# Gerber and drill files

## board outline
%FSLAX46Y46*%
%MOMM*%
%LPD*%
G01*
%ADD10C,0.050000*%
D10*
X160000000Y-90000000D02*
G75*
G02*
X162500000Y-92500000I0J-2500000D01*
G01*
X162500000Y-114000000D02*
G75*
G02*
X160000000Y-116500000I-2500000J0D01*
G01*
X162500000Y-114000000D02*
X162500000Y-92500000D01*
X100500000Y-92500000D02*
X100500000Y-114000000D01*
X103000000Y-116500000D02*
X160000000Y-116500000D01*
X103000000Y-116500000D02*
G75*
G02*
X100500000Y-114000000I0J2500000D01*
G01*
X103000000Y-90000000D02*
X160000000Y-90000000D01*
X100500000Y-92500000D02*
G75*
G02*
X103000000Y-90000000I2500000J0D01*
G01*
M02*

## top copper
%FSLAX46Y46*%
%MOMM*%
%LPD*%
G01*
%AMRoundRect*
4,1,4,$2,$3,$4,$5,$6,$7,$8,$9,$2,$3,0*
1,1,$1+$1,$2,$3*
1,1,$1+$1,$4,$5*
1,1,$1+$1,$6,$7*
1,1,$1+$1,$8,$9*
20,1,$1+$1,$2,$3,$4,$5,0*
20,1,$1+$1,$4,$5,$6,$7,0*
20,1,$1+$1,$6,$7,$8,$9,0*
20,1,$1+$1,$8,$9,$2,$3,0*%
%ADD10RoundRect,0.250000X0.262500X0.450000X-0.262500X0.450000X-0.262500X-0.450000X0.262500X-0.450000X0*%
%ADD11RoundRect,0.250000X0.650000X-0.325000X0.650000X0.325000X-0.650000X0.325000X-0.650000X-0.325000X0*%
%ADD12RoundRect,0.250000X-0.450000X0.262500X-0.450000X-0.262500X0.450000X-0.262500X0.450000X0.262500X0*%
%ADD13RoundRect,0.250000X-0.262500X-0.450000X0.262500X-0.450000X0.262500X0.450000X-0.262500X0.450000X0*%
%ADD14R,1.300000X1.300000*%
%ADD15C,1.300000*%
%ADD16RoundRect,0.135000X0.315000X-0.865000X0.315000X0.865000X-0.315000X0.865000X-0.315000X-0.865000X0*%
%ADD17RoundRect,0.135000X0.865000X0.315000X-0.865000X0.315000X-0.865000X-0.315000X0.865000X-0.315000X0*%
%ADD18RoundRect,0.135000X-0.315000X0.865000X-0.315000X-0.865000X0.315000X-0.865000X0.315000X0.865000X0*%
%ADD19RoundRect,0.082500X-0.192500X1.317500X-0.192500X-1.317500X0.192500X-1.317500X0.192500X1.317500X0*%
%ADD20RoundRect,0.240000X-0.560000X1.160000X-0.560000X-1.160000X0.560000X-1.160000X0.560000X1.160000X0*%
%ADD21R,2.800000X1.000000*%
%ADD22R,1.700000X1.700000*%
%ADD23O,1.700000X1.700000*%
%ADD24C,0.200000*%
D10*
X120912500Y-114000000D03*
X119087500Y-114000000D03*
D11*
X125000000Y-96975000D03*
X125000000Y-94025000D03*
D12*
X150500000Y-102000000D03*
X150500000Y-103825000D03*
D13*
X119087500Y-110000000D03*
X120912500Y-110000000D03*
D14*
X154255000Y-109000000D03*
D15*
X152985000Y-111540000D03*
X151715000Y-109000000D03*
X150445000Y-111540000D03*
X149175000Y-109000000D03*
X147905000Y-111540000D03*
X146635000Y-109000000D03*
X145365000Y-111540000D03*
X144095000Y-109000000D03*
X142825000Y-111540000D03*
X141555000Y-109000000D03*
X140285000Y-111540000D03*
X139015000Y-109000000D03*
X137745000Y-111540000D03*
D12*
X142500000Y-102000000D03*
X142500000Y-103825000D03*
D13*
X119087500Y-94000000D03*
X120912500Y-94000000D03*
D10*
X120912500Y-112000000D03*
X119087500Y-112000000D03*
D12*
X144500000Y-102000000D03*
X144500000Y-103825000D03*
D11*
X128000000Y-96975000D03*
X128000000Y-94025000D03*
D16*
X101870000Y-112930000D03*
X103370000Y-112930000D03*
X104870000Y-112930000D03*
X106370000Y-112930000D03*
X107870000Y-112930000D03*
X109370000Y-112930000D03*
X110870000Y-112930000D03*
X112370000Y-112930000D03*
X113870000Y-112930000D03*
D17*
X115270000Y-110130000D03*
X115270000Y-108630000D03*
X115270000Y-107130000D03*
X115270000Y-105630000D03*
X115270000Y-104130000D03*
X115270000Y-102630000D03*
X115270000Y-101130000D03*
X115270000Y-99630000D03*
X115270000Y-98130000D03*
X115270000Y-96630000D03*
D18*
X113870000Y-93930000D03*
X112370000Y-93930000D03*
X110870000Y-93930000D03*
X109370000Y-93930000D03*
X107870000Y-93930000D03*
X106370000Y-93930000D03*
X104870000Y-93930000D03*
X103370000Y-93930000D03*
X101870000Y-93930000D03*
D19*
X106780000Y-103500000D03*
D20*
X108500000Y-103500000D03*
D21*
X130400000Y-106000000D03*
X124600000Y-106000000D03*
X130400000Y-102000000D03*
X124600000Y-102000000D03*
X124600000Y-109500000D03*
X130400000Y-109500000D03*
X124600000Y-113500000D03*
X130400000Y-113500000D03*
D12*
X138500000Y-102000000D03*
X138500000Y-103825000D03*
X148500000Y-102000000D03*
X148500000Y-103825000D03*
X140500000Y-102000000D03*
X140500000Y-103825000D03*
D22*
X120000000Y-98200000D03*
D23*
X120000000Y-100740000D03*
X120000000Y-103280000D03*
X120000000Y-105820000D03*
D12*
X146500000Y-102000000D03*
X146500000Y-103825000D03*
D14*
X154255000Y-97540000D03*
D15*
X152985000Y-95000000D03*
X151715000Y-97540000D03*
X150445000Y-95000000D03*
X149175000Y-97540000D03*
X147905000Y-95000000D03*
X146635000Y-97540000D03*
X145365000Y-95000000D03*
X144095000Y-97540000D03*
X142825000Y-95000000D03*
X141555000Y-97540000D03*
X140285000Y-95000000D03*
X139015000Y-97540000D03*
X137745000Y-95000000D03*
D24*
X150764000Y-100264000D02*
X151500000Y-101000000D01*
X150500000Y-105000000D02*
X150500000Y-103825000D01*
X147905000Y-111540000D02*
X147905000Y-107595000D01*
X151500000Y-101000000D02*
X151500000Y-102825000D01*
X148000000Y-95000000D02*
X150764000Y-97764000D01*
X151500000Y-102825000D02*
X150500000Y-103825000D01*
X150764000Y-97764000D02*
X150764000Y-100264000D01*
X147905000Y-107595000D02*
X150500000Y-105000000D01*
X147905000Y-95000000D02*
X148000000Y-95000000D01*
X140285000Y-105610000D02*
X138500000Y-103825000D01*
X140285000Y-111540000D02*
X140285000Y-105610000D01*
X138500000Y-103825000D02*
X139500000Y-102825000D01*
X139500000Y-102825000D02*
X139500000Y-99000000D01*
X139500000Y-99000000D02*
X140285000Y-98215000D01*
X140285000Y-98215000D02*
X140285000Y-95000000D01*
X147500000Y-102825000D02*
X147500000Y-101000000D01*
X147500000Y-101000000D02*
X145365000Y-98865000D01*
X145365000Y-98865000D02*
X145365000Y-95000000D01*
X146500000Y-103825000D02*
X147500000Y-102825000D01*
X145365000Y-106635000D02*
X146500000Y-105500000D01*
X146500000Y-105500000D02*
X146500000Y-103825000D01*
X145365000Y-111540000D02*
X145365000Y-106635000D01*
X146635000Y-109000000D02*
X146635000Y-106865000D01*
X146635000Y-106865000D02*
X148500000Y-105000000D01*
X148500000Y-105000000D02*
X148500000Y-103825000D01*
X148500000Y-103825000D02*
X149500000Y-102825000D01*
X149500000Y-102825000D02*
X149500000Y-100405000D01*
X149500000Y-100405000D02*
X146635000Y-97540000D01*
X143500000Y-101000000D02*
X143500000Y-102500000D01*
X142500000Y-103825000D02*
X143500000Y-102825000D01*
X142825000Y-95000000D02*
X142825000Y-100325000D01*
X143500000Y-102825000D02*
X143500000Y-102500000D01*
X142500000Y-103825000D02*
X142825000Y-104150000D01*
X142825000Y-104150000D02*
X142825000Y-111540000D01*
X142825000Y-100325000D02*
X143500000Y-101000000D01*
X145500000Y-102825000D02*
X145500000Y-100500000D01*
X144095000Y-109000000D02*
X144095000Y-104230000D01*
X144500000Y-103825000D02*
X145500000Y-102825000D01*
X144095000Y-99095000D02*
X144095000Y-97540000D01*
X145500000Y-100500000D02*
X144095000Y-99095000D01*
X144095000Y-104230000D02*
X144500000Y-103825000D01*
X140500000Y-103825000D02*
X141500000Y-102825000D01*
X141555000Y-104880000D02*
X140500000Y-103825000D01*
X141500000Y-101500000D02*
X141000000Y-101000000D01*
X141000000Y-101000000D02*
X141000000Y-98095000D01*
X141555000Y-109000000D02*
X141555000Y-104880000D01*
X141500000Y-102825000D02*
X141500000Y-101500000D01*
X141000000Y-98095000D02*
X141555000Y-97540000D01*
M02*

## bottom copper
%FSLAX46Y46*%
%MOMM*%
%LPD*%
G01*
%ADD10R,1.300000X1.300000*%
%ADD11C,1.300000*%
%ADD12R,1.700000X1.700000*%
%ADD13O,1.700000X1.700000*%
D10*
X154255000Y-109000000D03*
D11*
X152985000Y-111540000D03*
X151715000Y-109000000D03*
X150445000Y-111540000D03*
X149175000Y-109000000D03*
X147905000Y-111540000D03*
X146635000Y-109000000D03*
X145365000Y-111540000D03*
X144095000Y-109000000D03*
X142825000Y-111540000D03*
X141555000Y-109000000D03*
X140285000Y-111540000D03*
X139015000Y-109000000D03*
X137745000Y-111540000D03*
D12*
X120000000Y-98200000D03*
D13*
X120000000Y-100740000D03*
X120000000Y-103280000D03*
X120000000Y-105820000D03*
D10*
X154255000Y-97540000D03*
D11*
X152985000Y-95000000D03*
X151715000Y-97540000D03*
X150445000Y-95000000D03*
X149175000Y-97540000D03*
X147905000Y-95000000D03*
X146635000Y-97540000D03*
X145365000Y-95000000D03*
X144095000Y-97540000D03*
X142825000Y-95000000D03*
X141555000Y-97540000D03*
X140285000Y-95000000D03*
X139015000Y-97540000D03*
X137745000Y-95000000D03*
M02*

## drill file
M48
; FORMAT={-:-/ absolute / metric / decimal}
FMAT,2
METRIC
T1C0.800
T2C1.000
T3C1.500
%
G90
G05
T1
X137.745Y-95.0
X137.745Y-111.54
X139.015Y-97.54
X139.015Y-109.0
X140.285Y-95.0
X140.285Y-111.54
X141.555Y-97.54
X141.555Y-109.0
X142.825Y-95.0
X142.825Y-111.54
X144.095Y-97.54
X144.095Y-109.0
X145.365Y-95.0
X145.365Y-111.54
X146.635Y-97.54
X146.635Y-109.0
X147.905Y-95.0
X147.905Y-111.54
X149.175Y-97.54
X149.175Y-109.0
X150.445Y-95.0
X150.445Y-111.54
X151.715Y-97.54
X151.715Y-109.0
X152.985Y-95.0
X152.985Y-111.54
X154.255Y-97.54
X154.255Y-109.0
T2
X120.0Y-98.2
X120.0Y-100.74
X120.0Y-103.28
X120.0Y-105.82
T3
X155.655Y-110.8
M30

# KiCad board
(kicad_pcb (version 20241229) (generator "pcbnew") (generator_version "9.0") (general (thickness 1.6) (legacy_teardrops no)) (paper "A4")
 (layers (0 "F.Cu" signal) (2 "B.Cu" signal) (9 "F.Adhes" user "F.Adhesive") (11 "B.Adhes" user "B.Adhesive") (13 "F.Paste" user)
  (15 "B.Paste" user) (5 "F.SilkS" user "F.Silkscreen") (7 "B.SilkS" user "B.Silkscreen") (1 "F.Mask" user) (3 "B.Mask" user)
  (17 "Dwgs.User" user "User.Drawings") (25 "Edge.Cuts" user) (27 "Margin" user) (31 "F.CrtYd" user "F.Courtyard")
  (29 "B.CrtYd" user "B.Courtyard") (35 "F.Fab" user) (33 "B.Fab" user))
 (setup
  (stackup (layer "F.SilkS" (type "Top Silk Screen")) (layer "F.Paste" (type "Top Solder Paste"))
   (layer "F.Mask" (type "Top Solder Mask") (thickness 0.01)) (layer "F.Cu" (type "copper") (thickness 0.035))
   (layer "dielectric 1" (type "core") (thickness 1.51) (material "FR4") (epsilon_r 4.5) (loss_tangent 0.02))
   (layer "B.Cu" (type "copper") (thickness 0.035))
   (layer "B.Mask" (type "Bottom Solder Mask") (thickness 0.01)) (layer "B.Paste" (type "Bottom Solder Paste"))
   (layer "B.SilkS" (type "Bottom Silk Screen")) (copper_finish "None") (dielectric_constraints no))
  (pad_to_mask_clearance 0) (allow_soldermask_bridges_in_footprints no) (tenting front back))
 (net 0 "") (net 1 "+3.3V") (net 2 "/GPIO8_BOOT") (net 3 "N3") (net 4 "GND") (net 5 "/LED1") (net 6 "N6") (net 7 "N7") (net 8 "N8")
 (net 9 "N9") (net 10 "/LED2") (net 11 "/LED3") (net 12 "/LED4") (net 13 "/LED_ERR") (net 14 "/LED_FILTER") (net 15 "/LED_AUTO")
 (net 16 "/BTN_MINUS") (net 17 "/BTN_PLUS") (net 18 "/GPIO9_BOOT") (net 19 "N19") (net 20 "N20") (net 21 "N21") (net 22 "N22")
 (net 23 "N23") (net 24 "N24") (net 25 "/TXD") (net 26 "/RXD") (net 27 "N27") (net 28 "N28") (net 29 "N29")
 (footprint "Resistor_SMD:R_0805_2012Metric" (layer "F.Cu") (at 120 114 180)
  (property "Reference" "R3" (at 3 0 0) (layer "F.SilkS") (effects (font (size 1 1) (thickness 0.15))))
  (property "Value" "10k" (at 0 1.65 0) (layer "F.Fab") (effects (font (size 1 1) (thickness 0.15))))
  (pad "1" smd roundrect (at -0.9125 0 180) (size 1.025 1.4) (layers "F.Cu" "F.Mask" "F.Paste") (roundrect_rratio 0.243902) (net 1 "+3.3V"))
  (pad "2" smd roundrect (at 0.9125 0 180) (size 1.025 1.4) (layers "F.Cu" "F.Mask" "F.Paste") (roundrect_rratio 0.243902)
   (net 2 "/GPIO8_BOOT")))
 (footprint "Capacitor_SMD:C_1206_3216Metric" (layer "F.Cu") (at 125 95.5 90)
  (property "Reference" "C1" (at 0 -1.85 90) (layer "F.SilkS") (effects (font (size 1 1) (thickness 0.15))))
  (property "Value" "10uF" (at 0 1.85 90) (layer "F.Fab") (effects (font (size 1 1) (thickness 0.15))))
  (pad "1" smd roundrect (at -1.475 0 90) (size 1.15 1.8) (layers "F.Cu" "F.Mask" "F.Paste") (roundrect_rratio 0.217391) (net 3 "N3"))
  (pad "2" smd roundrect (at 1.475 0 90) (size 1.15 1.8) (layers "F.Cu" "F.Mask" "F.Paste") (roundrect_rratio 0.217391) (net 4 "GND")))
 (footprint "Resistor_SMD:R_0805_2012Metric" (layer "F.Cu") (at 150.5 102.9125 -90)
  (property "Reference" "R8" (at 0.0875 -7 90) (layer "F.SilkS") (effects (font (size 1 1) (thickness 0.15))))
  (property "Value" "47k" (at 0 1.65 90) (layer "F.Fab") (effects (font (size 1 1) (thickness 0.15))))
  (pad "1" smd roundrect (at -0.9125 0 270) (size 1.025 1.4) (layers "F.Cu" "F.Mask" "F.Paste") (roundrect_rratio 0.243902) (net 1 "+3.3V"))
  (pad "2" smd roundrect (at 0.9125 0 270) (size 1.025 1.4) (layers "F.Cu" "F.Mask" "F.Paste") (roundrect_rratio 0.243902) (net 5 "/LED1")))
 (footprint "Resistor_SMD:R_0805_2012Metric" (layer "F.Cu") (at 120 110)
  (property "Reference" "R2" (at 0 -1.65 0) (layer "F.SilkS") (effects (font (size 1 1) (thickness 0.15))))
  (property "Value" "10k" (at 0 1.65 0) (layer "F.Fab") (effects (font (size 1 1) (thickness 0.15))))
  (pad "1" smd roundrect (at -0.9125 0) (size 1.025 1.4) (layers "F.Cu" "F.Mask" "F.Paste") (roundrect_rratio 0.243902) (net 1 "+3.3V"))
  (pad "2" smd roundrect (at 0.9125 0) (size 1.025 1.4) (layers "F.Cu" "F.Mask" "F.Paste") (roundrect_rratio 0.243902) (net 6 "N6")))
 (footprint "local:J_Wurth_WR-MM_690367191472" (layer "F.Cu") (at 154.255 109 -90)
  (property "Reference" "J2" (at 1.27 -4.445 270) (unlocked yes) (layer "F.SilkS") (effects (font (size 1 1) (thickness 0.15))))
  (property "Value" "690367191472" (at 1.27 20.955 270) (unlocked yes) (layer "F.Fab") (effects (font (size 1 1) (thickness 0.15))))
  (pad "" np_thru_hole circle (at 1.8 -1.4) (size 1.5 1.5) (drill 1.5) (layers "*.Cu" "*.Mask"))
  (pad "1" thru_hole rect (at 0 0) (size 1.3 1.3) (drill 0.8) (layers "*.Cu" "*.Mask") (remove_unused_layers no) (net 1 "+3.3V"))
  (pad "2" thru_hole circle (at 2.54 1.27) (size 1.3 1.3) (drill 0.8) (layers "*.Cu" "*.Mask") (remove_unused_layers no) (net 4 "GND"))
  (pad "3" thru_hole circle (at 0 2.54) (size 1.3 1.3) (drill 0.8) (layers "*.Cu" "*.Mask") (remove_unused_layers no) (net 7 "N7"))
  (pad "4" thru_hole circle (at 2.54 3.81) (size 1.3 1.3) (drill 0.8) (layers "*.Cu" "*.Mask") (remove_unused_layers no) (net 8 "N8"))
  (pad "5" thru_hole circle (at 0 5.08) (size 1.3 1.3) (drill 0.8) (layers "*.Cu" "*.Mask") (remove_unused_layers no) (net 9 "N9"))
  (pad "6" thru_hole circle (at 2.54 6.35) (size 1.3 1.3) (drill 0.8) (layers "*.Cu" "*.Mask") (remove_unused_layers no) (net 5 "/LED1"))
  (pad "7" thru_hole circle (at 0 7.62) (size 1.3 1.3) (drill 0.8) (layers "*.Cu" "*.Mask") (remove_unused_layers no) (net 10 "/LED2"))
  (pad "8" thru_hole circle (at 2.54 8.89) (size 1.3 1.3) (drill 0.8) (layers "*.Cu" "*.Mask") (remove_unused_layers no) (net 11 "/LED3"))
  (pad "9" thru_hole circle (at 0 10.16) (size 1.3 1.3) (drill 0.8) (layers "*.Cu" "*.Mask") (remove_unused_layers no) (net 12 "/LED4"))
  (pad "10" thru_hole circle (at 2.54 11.43) (size 1.3 1.3) (drill 0.8) (layers "*.Cu" "*.Mask") (remove_unused_layers no)
   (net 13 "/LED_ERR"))
  (pad "11" thru_hole circle (at 0 12.7) (size 1.3 1.3) (drill 0.8) (layers "*.Cu" "*.Mask") (remove_unused_layers no)
   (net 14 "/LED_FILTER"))
  (pad "12" thru_hole circle (at 2.54 13.97) (size 1.3 1.3) (drill 0.8) (layers "*.Cu" "*.Mask") (remove_unused_layers no)
   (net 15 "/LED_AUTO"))
  (pad "13" thru_hole circle (at 0 15.24) (size 1.3 1.3) (drill 0.8) (layers "*.Cu" "*.Mask") (remove_unused_layers no)
   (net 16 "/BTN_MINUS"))
  (pad "14" thru_hole circle (at 2.54 16.51) (size 1.3 1.3) (drill 0.8) (layers "*.Cu" "*.Mask") (remove_unused_layers no)
   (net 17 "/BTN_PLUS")))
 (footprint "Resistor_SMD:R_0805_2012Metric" (layer "F.Cu") (at 142.5 102.9125 -90)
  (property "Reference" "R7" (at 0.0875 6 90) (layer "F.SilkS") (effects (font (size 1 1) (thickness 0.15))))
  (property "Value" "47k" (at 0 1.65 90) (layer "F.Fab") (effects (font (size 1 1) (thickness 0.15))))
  (pad "1" smd roundrect (at -0.9125 0 270) (size 1.025 1.4) (layers "F.Cu" "F.Mask" "F.Paste") (roundrect_rratio 0.243902) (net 1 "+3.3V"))
  (pad "2" smd roundrect (at 0.9125 0 270) (size 1.025 1.4) (layers "F.Cu" "F.Mask" "F.Paste") (roundrect_rratio 0.243902)
   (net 13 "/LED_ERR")))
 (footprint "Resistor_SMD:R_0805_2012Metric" (layer "F.Cu") (at 120 94)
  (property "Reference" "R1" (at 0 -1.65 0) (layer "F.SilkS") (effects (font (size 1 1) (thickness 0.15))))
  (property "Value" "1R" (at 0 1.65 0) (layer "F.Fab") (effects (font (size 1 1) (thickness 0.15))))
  (pad "1" smd roundrect (at -0.9125 0) (size 1.025 1.4) (layers "F.Cu" "F.Mask" "F.Paste") (roundrect_rratio 0.243902) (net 1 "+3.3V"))
  (pad "2" smd roundrect (at 0.9125 0) (size 1.025 1.4) (layers "F.Cu" "F.Mask" "F.Paste") (roundrect_rratio 0.243902) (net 3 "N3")))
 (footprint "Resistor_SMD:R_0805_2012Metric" (layer "F.Cu") (at 120 112 180)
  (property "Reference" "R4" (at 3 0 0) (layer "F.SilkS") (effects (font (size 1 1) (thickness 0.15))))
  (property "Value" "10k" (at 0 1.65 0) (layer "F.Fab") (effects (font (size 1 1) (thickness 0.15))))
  (pad "1" smd roundrect (at -0.9125 0 180) (size 1.025 1.4) (layers "F.Cu" "F.Mask" "F.Paste") (roundrect_rratio 0.243902) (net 1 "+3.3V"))
  (pad "2" smd roundrect (at 0.9125 0 180) (size 1.025 1.4) (layers "F.Cu" "F.Mask" "F.Paste") (roundrect_rratio 0.243902)
   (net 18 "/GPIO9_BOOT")))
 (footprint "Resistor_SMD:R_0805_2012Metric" (layer "F.Cu") (at 144.5 102.9125 -90)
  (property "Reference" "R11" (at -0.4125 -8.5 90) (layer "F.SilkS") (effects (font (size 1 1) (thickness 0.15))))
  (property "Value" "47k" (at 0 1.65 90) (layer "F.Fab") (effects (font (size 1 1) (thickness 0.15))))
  (pad "1" smd roundrect (at -0.9125 0 270) (size 1.025 1.4) (layers "F.Cu" "F.Mask" "F.Paste") (roundrect_rratio 0.243902) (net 1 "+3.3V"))
  (pad "2" smd roundrect (at 0.9125 0 270) (size 1.025 1.4) (layers "F.Cu" "F.Mask" "F.Paste") (roundrect_rratio 0.243902) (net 12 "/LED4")))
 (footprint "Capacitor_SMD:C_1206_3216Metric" (layer "F.Cu") (at 128 95.5 90)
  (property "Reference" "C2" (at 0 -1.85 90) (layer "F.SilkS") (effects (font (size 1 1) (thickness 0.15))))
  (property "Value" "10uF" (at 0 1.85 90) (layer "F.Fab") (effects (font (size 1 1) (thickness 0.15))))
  (pad "1" smd roundrect (at -1.475 0 90) (size 1.15 1.8) (layers "F.Cu" "F.Mask" "F.Paste") (roundrect_rratio 0.217391) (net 3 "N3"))
  (pad "2" smd roundrect (at 1.475 0 90) (size 1.15 1.8) (layers "F.Cu" "F.Mask" "F.Paste") (roundrect_rratio 0.217391) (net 4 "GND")))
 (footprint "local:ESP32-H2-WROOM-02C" (layer "F.Cu") (at 107.87 103.43 90)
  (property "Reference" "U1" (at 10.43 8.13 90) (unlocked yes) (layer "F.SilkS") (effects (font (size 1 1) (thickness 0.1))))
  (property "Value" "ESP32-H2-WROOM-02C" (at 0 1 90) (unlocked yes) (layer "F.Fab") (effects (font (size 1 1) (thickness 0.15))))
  (pad "1" smd roundrect (at -9.5 -6 90) (size 2 0.9) (layers "F.Cu" "F.Mask" "F.Paste") (roundrect_rratio 0.15) (thermal_bridge_angle 45))
  (pad "2" smd roundrect (at -9.5 -4.5 90) (size 2 0.9) (layers "F.Cu" "F.Mask" "F.Paste") (roundrect_rratio 0.15) (thermal_bridge_angle 45))
  (pad "3" smd roundrect (at -9.5 -3 90) (size 2 0.9) (layers "F.Cu" "F.Mask" "F.Paste") (roundrect_rratio 0.15) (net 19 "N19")
   (thermal_bridge_angle 45))
  (pad "4" smd roundrect (at -9.5 -1.5 90) (size 2 0.9) (layers "F.Cu" "F.Mask" "F.Paste") (roundrect_rratio 0.15) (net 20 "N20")
   (thermal_bridge_angle 45))
  (pad "5" smd roundrect (at -9.5 0 90) (size 2 0.9) (layers "F.Cu" "F.Mask" "F.Paste") (roundrect_rratio 0.15) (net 15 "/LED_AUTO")
   (thermal_bridge_angle 45))
  (pad "6" smd roundrect (at -9.5 1.5 90) (size 2 0.9) (layers "F.Cu" "F.Mask" "F.Paste") (roundrect_rratio 0.15) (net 14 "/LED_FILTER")
   (thermal_bridge_angle 45))
  (pad "7" smd roundrect (at -9.5 3 90) (size 2 0.9) (layers "F.Cu" "F.Mask" "F.Paste") (roundrect_rratio 0.15) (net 2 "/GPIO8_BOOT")
   (thermal_bridge_angle 45))
  (pad "8" smd roundrect (at -9.5 4.5 90) (size 2 0.9) (layers "F.Cu" "F.Mask" "F.Paste") (roundrect_rratio 0.15) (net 18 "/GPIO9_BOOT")
   (thermal_bridge_angle 45))
  (pad "9" smd roundrect (at -9.5 6 90) (size 2 0.9) (layers "F.Cu" "F.Mask" "F.Paste") (roundrect_rratio 0.15) (thermal_bridge_angle 45))
  (pad "10" smd roundrect (at -6.7 7.4 180) (size 2 0.9) (layers "F.Cu" "F.Mask" "F.Paste") (roundrect_rratio 0.15) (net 13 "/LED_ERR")
   (thermal_bridge_angle 45))
  (pad "11" smd roundrect (at -5.2 7.4 180) (size 2 0.9) (layers "F.Cu" "F.Mask" "F.Paste") (roundrect_rratio 0.15) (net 5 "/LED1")
   (thermal_bridge_angle 45))
  (pad "12" smd roundrect (at -3.7 7.4 180) (size 2 0.9) (layers "F.Cu" "F.Mask" "F.Paste") (roundrect_rratio 0.15) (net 10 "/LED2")
   (thermal_bridge_angle 45))
  (pad "13" smd roundrect (at -2.2 7.4 180) (size 2 0.9) (layers "F.Cu" "F.Mask" "F.Paste") (roundrect_rratio 0.15)
   (thermal_bridge_angle 45))
  (pad "14" smd roundrect (at -0.7 7.4 180) (size 2 0.9) (layers "F.Cu" "F.Mask" "F.Paste") (roundrect_rratio 0.15)
   (thermal_bridge_angle 45))
  (pad "15" smd roundrect (at 0.8 7.4 180) (size 2 0.9) (layers "F.Cu" "F.Mask" "F.Paste") (roundrect_rratio 0.15) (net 11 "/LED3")
   (thermal_bridge_angle 45))
  (pad "16" smd roundrect (at 2.3 7.4 180) (size 2 0.9) (layers "F.Cu" "F.Mask" "F.Paste") (roundrect_rratio 0.15) (thermal_bridge_angle 45))
  (pad "17" smd roundrect (at 3.8 7.4 180) (size 2 0.9) (layers "F.Cu" "F.Mask" "F.Paste") (roundrect_rratio 0.15) (thermal_bridge_angle 45))
  (pad "18" smd roundrect (at 5.3 7.4 180) (size 2 0.9) (layers "F.Cu" "F.Mask" "F.Paste") (roundrect_rratio 0.15) (thermal_bridge_angle 45))
  (pad "19" smd roundrect (at 6.8 7.4 180) (size 2 0.9) (layers "F.Cu" "F.Mask" "F.Paste") (roundrect_rratio 0.15) (thermal_bridge_angle 45))
  (pad "20" smd roundrect (at 9.5 6 270) (size 2 0.9) (layers "F.Cu" "F.Mask" "F.Paste") (roundrect_rratio 0.15) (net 12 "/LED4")
   (thermal_bridge_angle 45))
  (pad "21" smd roundrect (at 9.5 4.5 270) (size 2 0.9) (layers "F.Cu" "F.Mask" "F.Paste") (roundrect_rratio 0.15) (thermal_bridge_angle 45))
  (pad "22" smd roundrect (at 9.5 3 270) (size 2 0.9) (layers "F.Cu" "F.Mask" "F.Paste") (roundrect_rratio 0.15) (thermal_bridge_angle 45))
  (pad "23" smd roundrect (at 9.5 1.5 270) (size 2 0.9) (layers "F.Cu" "F.Mask" "F.Paste") (roundrect_rratio 0.15) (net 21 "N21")
   (thermal_bridge_angle 45))
  (pad "24" smd roundrect (at 9.5 0 270) (size 2 0.9) (layers "F.Cu" "F.Mask" "F.Paste") (roundrect_rratio 0.15) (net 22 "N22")
   (thermal_bridge_angle 45))
  (pad "25" smd roundrect (at 9.5 -1.5 270) (size 2 0.9) (layers "F.Cu" "F.Mask" "F.Paste") (roundrect_rratio 0.15) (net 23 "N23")
   (thermal_bridge_angle 45))
  (pad "26" smd roundrect (at 9.5 -3 270) (size 2 0.9) (layers "F.Cu" "F.Mask" "F.Paste") (roundrect_rratio 0.15) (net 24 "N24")
   (thermal_bridge_angle 45))
  (pad "27" smd roundrect (at 9.5 -4.5 270) (size 2 0.9) (layers "F.Cu" "F.Mask" "F.Paste") (roundrect_rratio 0.15) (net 16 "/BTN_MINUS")
   (thermal_bridge_angle 45))
  (pad "28" smd roundrect (at 9.5 -6 270) (size 2 0.9) (layers "F.Cu" "F.Mask" "F.Paste") (roundrect_rratio 0.15) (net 17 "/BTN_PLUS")
   (thermal_bridge_angle 45))
  (pad "29" smd roundrect (at -0.07 -1.09 270) (size 2.8 0.55) (layers "F.Cu" "F.Mask" "F.Paste") (roundrect_rratio 0.15)
   (thermal_bridge_angle 45))
  (pad "30" smd roundrect (at -0.07 0.63 270) (size 2.8 1.6) (layers "F.Cu" "F.Mask" "F.Paste") (roundrect_rratio 0.15)
   (thermal_bridge_angle 45)))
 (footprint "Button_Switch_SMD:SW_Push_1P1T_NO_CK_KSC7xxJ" (layer "F.Cu") (at 127.5 104 180)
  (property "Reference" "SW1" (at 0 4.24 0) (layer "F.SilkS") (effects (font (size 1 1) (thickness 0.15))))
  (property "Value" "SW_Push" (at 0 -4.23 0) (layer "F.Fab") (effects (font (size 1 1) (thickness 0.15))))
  (pad "1" smd rect (at -2.9 -2 180) (size 2.8 1) (layers "F.Cu" "F.Mask" "F.Paste") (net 4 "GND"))
  (pad "1" smd rect (at 2.9 -2 180) (size 2.8 1) (layers "F.Cu" "F.Mask" "F.Paste") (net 4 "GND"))
  (pad "2" smd rect (at -2.9 2 180) (size 2.8 1) (layers "F.Cu" "F.Mask" "F.Paste") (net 6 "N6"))
  (pad "2" smd rect (at 2.9 2 180) (size 2.8 1) (layers "F.Cu" "F.Mask" "F.Paste") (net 6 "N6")))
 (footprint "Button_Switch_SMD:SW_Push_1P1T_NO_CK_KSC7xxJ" (layer "F.Cu") (at 127.5 111.5)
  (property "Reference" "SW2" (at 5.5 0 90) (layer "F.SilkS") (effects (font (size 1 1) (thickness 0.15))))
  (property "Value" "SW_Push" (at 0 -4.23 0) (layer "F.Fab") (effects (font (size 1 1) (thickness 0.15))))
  (pad "1" smd rect (at -2.9 -2) (size 2.8 1) (layers "F.Cu" "F.Mask" "F.Paste") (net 4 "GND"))
  (pad "1" smd rect (at 2.9 -2) (size 2.8 1) (layers "F.Cu" "F.Mask" "F.Paste") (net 4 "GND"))
  (pad "2" smd rect (at -2.9 2) (size 2.8 1) (layers "F.Cu" "F.Mask" "F.Paste") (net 18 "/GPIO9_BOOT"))
  (pad "2" smd rect (at 2.9 2) (size 2.8 1) (layers "F.Cu" "F.Mask" "F.Paste") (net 18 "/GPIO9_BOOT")))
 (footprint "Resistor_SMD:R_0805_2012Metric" (layer "F.Cu") (at 138.5 102.9125 -90)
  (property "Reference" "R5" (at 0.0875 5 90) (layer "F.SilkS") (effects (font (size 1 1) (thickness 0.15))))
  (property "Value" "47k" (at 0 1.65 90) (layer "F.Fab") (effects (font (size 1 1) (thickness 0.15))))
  (pad "1" smd roundrect (at -0.9125 0 270) (size 1.025 1.4) (layers "F.Cu" "F.Mask" "F.Paste") (roundrect_rratio 0.243902) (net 1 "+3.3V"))
  (pad "2" smd roundrect (at 0.9125 0 270) (size 1.025 1.4) (layers "F.Cu" "F.Mask" "F.Paste") (roundrect_rratio 0.243902)
   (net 15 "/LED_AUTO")))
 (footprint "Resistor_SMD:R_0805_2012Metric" (layer "F.Cu") (at 148.5 102.9125 -90)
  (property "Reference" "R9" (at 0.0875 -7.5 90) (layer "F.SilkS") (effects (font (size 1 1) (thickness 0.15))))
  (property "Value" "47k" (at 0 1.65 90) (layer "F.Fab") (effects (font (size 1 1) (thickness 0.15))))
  (pad "1" smd roundrect (at -0.9125 0 270) (size 1.025 1.4) (layers "F.Cu" "F.Mask" "F.Paste") (roundrect_rratio 0.243902) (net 1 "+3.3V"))
  (pad "2" smd roundrect (at 0.9125 0 270) (size 1.025 1.4) (layers "F.Cu" "F.Mask" "F.Paste") (roundrect_rratio 0.243902) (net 10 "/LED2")))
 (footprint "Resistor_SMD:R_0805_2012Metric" (layer "F.Cu") (at 140.5 102.9125 -90)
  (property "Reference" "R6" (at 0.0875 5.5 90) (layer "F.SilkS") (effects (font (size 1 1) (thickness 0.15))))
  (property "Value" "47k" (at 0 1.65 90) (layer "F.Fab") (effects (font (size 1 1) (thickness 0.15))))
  (pad "1" smd roundrect (at -0.9125 0 270) (size 1.025 1.4) (layers "F.Cu" "F.Mask" "F.Paste") (roundrect_rratio 0.243902) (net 1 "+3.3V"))
  (pad "2" smd roundrect (at 0.9125 0 270) (size 1.025 1.4) (layers "F.Cu" "F.Mask" "F.Paste") (roundrect_rratio 0.243902)
   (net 14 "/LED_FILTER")))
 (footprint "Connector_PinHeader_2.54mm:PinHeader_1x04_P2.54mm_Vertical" (layer "F.Cu") (at 120 98.2)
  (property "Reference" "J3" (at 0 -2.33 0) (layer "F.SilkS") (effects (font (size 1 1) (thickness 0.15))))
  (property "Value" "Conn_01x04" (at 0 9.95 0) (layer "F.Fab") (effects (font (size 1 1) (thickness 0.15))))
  (pad "1" thru_hole rect (at 0 0) (size 1.7 1.7) (drill 1) (layers "*.Cu" "*.Mask") (remove_unused_layers no) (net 1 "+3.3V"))
  (pad "2" thru_hole oval (at 0 2.54) (size 1.7 1.7) (drill 1) (layers "*.Cu" "*.Mask") (remove_unused_layers no) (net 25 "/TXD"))
  (pad "3" thru_hole oval (at 0 5.08) (size 1.7 1.7) (drill 1) (layers "*.Cu" "*.Mask") (remove_unused_layers no) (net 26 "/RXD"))
  (pad "4" thru_hole oval (at 0 7.62) (size 1.7 1.7) (drill 1) (layers "*.Cu" "*.Mask") (remove_unused_layers no) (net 4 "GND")))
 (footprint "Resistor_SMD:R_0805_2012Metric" (layer "F.Cu") (at 146.5 102.9125 -90)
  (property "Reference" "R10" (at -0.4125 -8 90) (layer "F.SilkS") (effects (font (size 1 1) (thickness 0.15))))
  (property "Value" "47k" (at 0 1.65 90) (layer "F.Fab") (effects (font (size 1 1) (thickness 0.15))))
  (pad "1" smd roundrect (at -0.9125 0 270) (size 1.025 1.4) (layers "F.Cu" "F.Mask" "F.Paste") (roundrect_rratio 0.243902) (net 1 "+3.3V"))
  (pad "2" smd roundrect (at 0.9125 0 270) (size 1.025 1.4) (layers "F.Cu" "F.Mask" "F.Paste") (roundrect_rratio 0.243902) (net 11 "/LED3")))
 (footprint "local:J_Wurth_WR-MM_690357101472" (layer "B.Cu") (at 154.255 97.54 90)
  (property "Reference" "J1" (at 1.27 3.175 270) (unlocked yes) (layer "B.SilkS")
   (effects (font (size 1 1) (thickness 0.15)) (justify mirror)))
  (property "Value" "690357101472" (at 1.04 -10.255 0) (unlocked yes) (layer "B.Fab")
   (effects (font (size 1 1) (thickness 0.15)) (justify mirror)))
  (pad "1" thru_hole rect (at 0 0) (size 1.3 1.3) (drill 0.8) (layers "*.Cu" "*.Mask") (remove_unused_layers no) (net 1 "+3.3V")
   (thermal_bridge_angle 45))
  (pad "2" thru_hole circle (at 2.54 -1.27) (size 1.3 1.3) (drill 0.8) (layers "*.Cu" "*.Mask") (remove_unused_layers no) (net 4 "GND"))
  (pad "3" thru_hole circle (at 0 -2.54) (size 1.3 1.3) (drill 0.8) (layers "*.Cu" "*.Mask") (remove_unused_layers no) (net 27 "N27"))
  (pad "4" thru_hole circle (at 2.54 -3.81) (size 1.3 1.3) (drill 0.8) (layers "*.Cu" "*.Mask") (remove_unused_layers no) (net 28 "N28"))
  (pad "5" thru_hole circle (at 0 -5.08) (size 1.3 1.3) (drill 0.8) (layers "*.Cu" "*.Mask") (remove_unused_layers no) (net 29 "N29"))
  (pad "6" thru_hole circle (at 2.54 -6.35) (size 1.3 1.3) (drill 0.8) (layers "*.Cu" "*.Mask") (remove_unused_layers no) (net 5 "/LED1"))
  (pad "7" thru_hole circle (at 0 -7.62) (size 1.3 1.3) (drill 0.8) (layers "*.Cu" "*.Mask") (remove_unused_layers no) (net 10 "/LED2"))
  (pad "8" thru_hole circle (at 2.54 -8.89) (size 1.3 1.3) (drill 0.8) (layers "*.Cu" "*.Mask") (remove_unused_layers no) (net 11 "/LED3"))
  (pad "9" thru_hole circle (at 0 -10.16) (size 1.3 1.3) (drill 0.8) (layers "*.Cu" "*.Mask") (remove_unused_layers no) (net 12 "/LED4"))
  (pad "10" thru_hole circle (at 2.54 -11.43) (size 1.3 1.3) (drill 0.8) (layers "*.Cu" "*.Mask") (remove_unused_layers no)
   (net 13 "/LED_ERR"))
  (pad "11" thru_hole circle (at 0 -12.7) (size 1.3 1.3) (drill 0.8) (layers "*.Cu" "*.Mask") (remove_unused_layers no)
   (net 14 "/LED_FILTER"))
  (pad "12" thru_hole circle (at 2.54 -13.97) (size 1.3 1.3) (drill 0.8) (layers "*.Cu" "*.Mask") (remove_unused_layers no)
   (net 15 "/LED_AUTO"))
  (pad "13" thru_hole circle (at 0 -15.24) (size 1.3 1.3) (drill 0.8) (layers "*.Cu" "*.Mask") (remove_unused_layers no)
   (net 16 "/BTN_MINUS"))
  (pad "14" thru_hole circle (at 2.54 -16.51) (size 1.3 1.3) (drill 0.8) (layers "*.Cu" "*.Mask") (remove_unused_layers no)
   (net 17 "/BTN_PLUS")))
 (gr_arc (start 160 90) (mid 161.767767 90.732233) (end 162.5 92.5) (stroke (width 0.05) (type default)) (locked yes) (layer "Edge.Cuts"))
 (gr_arc (start 162.5 114) (mid 161.767767 115.767767) (end 160 116.5) (stroke (width 0.05) (type default)) (locked yes) (layer "Edge.Cuts"))
 (gr_line (start 162.5 114) (end 162.5 92.5) (stroke (width 0.05) (type default)) (locked yes) (layer "Edge.Cuts"))
 (gr_line (start 100.5 92.5) (end 100.5 114) (stroke (width 0.05) (type default)) (locked yes) (layer "Edge.Cuts"))
 (gr_line (start 103 116.5) (end 160 116.5) (stroke (width 0.05) (type default)) (locked yes) (layer "Edge.Cuts"))
 (gr_arc (start 103 116.5) (mid 101.232233 115.767767) (end 100.5 114) (stroke (width 0.05) (type default)) (locked yes) (layer "Edge.Cuts"))
 (gr_line (start 103 90) (end 160 90) (stroke (width 0.05) (type default)) (locked yes) (layer "Edge.Cuts"))
 (gr_arc (start 100.5 92.5) (mid 101.232233 90.732233) (end 103 90) (stroke (width 0.05) (type default)) (locked yes) (layer "Edge.Cuts"))
 (segment (start 150.764 100.264) (end 151.5 101) (width 0.2) (layer "F.Cu") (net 5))
 (segment (start 150.5 105) (end 150.5 103.825) (width 0.2) (layer "F.Cu") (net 5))
 (segment (start 147.905 111.54) (end 147.905 107.595) (width 0.2) (layer "F.Cu") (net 5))
 (segment (start 151.5 101) (end 151.5 102.825) (width 0.2) (layer "F.Cu") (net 5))
 (segment (start 148 95) (end 150.764 97.764) (width 0.2) (layer "F.Cu") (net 5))
 (segment (start 151.5 102.825) (end 150.5 103.825) (width 0.2) (layer "F.Cu") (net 5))
 (segment (start 150.764 97.764) (end 150.764 100.264) (width 0.2) (layer "F.Cu") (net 5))
 (segment (start 147.905 107.595) (end 150.5 105) (width 0.2) (layer "F.Cu") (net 5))
 (segment (start 147.905 95) (end 148 95) (width 0.2) (layer "F.Cu") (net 5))
 (segment (start 140.285 105.61) (end 138.5 103.825) (width 0.2) (layer "F.Cu") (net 15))
 (segment (start 140.285 111.54) (end 140.285 105.61) (width 0.2) (layer "F.Cu") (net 15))
 (segment (start 138.5 103.825) (end 139.5 102.825) (width 0.2) (layer "F.Cu") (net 15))
 (segment (start 139.5 102.825) (end 139.5 99) (width 0.2) (layer "F.Cu") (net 15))
 (segment (start 139.5 99) (end 140.285 98.215) (width 0.2) (layer "F.Cu") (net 15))
 (segment (start 140.285 98.215) (end 140.285 95) (width 0.2) (layer "F.Cu") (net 15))
 (segment (start 147.5 102.825) (end 147.5 101) (width 0.2) (layer "F.Cu") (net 11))
 (segment (start 147.5 101) (end 145.365 98.865) (width 0.2) (layer "F.Cu") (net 11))
 (segment (start 145.365 98.865) (end 145.365 95) (width 0.2) (layer "F.Cu") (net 11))
 (segment (start 146.5 103.825) (end 147.5 102.825) (width 0.2) (layer "F.Cu") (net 11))
 (segment (start 145.365 106.635) (end 146.5 105.5) (width 0.2) (layer "F.Cu") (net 11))
 (segment (start 146.5 105.5) (end 146.5 103.825) (width 0.2) (layer "F.Cu") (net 11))
 (segment (start 145.365 111.54) (end 145.365 106.635) (width 0.2) (layer "F.Cu") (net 11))
 (segment (start 146.635 109) (end 146.635 106.865) (width 0.2) (layer "F.Cu") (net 10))
 (segment (start 146.635 106.865) (end 148.5 105) (width 0.2) (layer "F.Cu") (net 10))
 (segment (start 148.5 105) (end 148.5 103.825) (width 0.2) (layer "F.Cu") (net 10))
 (segment (start 148.5 103.825) (end 149.5 102.825) (width 0.2) (layer "F.Cu") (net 10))
 (segment (start 149.5 102.825) (end 149.5 100.405) (width 0.2) (layer "F.Cu") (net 10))
 (segment (start 149.5 100.405) (end 146.635 97.54) (width 0.2) (layer "F.Cu") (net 10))
 (segment (start 143.5 101) (end 143.5 102.5) (width 0.2) (layer "F.Cu") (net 13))
 (segment (start 142.5 103.825) (end 143.5 102.825) (width 0.2) (layer "F.Cu") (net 13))
 (segment (start 142.825 95) (end 142.825 100.325) (width 0.2) (layer "F.Cu") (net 13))
 (segment (start 143.5 102.825) (end 143.5 102.5) (width 0.2) (layer "F.Cu") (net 13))
 (segment (start 142.5 103.825) (end 142.825 104.15) (width 0.2) (layer "F.Cu") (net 13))
 (segment (start 142.825 104.15) (end 142.825 111.54) (width 0.2) (layer "F.Cu") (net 13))
 (segment (start 142.825 100.325) (end 143.5 101) (width 0.2) (layer "F.Cu") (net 13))
 (segment (start 145.5 102.825) (end 145.5 100.5) (width 0.2) (layer "F.Cu") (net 12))
 (segment (start 144.095 109) (end 144.095 104.23) (width 0.2) (layer "F.Cu") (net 12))
 (segment (start 144.5 103.825) (end 145.5 102.825) (width 0.2) (layer "F.Cu") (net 12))
 (segment (start 144.095 99.095) (end 144.095 97.54) (width 0.2) (layer "F.Cu") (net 12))
 (segment (start 145.5 100.5) (end 144.095 99.095) (width 0.2) (layer "F.Cu") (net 12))
 (segment (start 144.095 104.23) (end 144.5 103.825) (width 0.2) (layer "F.Cu") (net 12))
 (segment (start 140.5 103.825) (end 141.5 102.825) (width 0.2) (layer "F.Cu") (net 14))
 (segment (start 141.555 104.88) (end 140.5 103.825) (width 0.2) (layer "F.Cu") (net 14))
 (segment (start 141.5 101.5) (end 141 101) (width 0.2) (layer "F.Cu") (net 14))
 (segment (start 141 101) (end 141 98.095) (width 0.2) (layer "F.Cu") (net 14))
 (segment (start 141.555 109) (end 141.555 104.88) (width 0.2) (layer "F.Cu") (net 14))
 (segment (start 141.5 102.825) (end 141.5 101.5) (width 0.2) (layer "F.Cu") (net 14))
 (segment (start 141 98.095) (end 141.555 97.54) (width 0.2) (layer "F.Cu") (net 14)))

